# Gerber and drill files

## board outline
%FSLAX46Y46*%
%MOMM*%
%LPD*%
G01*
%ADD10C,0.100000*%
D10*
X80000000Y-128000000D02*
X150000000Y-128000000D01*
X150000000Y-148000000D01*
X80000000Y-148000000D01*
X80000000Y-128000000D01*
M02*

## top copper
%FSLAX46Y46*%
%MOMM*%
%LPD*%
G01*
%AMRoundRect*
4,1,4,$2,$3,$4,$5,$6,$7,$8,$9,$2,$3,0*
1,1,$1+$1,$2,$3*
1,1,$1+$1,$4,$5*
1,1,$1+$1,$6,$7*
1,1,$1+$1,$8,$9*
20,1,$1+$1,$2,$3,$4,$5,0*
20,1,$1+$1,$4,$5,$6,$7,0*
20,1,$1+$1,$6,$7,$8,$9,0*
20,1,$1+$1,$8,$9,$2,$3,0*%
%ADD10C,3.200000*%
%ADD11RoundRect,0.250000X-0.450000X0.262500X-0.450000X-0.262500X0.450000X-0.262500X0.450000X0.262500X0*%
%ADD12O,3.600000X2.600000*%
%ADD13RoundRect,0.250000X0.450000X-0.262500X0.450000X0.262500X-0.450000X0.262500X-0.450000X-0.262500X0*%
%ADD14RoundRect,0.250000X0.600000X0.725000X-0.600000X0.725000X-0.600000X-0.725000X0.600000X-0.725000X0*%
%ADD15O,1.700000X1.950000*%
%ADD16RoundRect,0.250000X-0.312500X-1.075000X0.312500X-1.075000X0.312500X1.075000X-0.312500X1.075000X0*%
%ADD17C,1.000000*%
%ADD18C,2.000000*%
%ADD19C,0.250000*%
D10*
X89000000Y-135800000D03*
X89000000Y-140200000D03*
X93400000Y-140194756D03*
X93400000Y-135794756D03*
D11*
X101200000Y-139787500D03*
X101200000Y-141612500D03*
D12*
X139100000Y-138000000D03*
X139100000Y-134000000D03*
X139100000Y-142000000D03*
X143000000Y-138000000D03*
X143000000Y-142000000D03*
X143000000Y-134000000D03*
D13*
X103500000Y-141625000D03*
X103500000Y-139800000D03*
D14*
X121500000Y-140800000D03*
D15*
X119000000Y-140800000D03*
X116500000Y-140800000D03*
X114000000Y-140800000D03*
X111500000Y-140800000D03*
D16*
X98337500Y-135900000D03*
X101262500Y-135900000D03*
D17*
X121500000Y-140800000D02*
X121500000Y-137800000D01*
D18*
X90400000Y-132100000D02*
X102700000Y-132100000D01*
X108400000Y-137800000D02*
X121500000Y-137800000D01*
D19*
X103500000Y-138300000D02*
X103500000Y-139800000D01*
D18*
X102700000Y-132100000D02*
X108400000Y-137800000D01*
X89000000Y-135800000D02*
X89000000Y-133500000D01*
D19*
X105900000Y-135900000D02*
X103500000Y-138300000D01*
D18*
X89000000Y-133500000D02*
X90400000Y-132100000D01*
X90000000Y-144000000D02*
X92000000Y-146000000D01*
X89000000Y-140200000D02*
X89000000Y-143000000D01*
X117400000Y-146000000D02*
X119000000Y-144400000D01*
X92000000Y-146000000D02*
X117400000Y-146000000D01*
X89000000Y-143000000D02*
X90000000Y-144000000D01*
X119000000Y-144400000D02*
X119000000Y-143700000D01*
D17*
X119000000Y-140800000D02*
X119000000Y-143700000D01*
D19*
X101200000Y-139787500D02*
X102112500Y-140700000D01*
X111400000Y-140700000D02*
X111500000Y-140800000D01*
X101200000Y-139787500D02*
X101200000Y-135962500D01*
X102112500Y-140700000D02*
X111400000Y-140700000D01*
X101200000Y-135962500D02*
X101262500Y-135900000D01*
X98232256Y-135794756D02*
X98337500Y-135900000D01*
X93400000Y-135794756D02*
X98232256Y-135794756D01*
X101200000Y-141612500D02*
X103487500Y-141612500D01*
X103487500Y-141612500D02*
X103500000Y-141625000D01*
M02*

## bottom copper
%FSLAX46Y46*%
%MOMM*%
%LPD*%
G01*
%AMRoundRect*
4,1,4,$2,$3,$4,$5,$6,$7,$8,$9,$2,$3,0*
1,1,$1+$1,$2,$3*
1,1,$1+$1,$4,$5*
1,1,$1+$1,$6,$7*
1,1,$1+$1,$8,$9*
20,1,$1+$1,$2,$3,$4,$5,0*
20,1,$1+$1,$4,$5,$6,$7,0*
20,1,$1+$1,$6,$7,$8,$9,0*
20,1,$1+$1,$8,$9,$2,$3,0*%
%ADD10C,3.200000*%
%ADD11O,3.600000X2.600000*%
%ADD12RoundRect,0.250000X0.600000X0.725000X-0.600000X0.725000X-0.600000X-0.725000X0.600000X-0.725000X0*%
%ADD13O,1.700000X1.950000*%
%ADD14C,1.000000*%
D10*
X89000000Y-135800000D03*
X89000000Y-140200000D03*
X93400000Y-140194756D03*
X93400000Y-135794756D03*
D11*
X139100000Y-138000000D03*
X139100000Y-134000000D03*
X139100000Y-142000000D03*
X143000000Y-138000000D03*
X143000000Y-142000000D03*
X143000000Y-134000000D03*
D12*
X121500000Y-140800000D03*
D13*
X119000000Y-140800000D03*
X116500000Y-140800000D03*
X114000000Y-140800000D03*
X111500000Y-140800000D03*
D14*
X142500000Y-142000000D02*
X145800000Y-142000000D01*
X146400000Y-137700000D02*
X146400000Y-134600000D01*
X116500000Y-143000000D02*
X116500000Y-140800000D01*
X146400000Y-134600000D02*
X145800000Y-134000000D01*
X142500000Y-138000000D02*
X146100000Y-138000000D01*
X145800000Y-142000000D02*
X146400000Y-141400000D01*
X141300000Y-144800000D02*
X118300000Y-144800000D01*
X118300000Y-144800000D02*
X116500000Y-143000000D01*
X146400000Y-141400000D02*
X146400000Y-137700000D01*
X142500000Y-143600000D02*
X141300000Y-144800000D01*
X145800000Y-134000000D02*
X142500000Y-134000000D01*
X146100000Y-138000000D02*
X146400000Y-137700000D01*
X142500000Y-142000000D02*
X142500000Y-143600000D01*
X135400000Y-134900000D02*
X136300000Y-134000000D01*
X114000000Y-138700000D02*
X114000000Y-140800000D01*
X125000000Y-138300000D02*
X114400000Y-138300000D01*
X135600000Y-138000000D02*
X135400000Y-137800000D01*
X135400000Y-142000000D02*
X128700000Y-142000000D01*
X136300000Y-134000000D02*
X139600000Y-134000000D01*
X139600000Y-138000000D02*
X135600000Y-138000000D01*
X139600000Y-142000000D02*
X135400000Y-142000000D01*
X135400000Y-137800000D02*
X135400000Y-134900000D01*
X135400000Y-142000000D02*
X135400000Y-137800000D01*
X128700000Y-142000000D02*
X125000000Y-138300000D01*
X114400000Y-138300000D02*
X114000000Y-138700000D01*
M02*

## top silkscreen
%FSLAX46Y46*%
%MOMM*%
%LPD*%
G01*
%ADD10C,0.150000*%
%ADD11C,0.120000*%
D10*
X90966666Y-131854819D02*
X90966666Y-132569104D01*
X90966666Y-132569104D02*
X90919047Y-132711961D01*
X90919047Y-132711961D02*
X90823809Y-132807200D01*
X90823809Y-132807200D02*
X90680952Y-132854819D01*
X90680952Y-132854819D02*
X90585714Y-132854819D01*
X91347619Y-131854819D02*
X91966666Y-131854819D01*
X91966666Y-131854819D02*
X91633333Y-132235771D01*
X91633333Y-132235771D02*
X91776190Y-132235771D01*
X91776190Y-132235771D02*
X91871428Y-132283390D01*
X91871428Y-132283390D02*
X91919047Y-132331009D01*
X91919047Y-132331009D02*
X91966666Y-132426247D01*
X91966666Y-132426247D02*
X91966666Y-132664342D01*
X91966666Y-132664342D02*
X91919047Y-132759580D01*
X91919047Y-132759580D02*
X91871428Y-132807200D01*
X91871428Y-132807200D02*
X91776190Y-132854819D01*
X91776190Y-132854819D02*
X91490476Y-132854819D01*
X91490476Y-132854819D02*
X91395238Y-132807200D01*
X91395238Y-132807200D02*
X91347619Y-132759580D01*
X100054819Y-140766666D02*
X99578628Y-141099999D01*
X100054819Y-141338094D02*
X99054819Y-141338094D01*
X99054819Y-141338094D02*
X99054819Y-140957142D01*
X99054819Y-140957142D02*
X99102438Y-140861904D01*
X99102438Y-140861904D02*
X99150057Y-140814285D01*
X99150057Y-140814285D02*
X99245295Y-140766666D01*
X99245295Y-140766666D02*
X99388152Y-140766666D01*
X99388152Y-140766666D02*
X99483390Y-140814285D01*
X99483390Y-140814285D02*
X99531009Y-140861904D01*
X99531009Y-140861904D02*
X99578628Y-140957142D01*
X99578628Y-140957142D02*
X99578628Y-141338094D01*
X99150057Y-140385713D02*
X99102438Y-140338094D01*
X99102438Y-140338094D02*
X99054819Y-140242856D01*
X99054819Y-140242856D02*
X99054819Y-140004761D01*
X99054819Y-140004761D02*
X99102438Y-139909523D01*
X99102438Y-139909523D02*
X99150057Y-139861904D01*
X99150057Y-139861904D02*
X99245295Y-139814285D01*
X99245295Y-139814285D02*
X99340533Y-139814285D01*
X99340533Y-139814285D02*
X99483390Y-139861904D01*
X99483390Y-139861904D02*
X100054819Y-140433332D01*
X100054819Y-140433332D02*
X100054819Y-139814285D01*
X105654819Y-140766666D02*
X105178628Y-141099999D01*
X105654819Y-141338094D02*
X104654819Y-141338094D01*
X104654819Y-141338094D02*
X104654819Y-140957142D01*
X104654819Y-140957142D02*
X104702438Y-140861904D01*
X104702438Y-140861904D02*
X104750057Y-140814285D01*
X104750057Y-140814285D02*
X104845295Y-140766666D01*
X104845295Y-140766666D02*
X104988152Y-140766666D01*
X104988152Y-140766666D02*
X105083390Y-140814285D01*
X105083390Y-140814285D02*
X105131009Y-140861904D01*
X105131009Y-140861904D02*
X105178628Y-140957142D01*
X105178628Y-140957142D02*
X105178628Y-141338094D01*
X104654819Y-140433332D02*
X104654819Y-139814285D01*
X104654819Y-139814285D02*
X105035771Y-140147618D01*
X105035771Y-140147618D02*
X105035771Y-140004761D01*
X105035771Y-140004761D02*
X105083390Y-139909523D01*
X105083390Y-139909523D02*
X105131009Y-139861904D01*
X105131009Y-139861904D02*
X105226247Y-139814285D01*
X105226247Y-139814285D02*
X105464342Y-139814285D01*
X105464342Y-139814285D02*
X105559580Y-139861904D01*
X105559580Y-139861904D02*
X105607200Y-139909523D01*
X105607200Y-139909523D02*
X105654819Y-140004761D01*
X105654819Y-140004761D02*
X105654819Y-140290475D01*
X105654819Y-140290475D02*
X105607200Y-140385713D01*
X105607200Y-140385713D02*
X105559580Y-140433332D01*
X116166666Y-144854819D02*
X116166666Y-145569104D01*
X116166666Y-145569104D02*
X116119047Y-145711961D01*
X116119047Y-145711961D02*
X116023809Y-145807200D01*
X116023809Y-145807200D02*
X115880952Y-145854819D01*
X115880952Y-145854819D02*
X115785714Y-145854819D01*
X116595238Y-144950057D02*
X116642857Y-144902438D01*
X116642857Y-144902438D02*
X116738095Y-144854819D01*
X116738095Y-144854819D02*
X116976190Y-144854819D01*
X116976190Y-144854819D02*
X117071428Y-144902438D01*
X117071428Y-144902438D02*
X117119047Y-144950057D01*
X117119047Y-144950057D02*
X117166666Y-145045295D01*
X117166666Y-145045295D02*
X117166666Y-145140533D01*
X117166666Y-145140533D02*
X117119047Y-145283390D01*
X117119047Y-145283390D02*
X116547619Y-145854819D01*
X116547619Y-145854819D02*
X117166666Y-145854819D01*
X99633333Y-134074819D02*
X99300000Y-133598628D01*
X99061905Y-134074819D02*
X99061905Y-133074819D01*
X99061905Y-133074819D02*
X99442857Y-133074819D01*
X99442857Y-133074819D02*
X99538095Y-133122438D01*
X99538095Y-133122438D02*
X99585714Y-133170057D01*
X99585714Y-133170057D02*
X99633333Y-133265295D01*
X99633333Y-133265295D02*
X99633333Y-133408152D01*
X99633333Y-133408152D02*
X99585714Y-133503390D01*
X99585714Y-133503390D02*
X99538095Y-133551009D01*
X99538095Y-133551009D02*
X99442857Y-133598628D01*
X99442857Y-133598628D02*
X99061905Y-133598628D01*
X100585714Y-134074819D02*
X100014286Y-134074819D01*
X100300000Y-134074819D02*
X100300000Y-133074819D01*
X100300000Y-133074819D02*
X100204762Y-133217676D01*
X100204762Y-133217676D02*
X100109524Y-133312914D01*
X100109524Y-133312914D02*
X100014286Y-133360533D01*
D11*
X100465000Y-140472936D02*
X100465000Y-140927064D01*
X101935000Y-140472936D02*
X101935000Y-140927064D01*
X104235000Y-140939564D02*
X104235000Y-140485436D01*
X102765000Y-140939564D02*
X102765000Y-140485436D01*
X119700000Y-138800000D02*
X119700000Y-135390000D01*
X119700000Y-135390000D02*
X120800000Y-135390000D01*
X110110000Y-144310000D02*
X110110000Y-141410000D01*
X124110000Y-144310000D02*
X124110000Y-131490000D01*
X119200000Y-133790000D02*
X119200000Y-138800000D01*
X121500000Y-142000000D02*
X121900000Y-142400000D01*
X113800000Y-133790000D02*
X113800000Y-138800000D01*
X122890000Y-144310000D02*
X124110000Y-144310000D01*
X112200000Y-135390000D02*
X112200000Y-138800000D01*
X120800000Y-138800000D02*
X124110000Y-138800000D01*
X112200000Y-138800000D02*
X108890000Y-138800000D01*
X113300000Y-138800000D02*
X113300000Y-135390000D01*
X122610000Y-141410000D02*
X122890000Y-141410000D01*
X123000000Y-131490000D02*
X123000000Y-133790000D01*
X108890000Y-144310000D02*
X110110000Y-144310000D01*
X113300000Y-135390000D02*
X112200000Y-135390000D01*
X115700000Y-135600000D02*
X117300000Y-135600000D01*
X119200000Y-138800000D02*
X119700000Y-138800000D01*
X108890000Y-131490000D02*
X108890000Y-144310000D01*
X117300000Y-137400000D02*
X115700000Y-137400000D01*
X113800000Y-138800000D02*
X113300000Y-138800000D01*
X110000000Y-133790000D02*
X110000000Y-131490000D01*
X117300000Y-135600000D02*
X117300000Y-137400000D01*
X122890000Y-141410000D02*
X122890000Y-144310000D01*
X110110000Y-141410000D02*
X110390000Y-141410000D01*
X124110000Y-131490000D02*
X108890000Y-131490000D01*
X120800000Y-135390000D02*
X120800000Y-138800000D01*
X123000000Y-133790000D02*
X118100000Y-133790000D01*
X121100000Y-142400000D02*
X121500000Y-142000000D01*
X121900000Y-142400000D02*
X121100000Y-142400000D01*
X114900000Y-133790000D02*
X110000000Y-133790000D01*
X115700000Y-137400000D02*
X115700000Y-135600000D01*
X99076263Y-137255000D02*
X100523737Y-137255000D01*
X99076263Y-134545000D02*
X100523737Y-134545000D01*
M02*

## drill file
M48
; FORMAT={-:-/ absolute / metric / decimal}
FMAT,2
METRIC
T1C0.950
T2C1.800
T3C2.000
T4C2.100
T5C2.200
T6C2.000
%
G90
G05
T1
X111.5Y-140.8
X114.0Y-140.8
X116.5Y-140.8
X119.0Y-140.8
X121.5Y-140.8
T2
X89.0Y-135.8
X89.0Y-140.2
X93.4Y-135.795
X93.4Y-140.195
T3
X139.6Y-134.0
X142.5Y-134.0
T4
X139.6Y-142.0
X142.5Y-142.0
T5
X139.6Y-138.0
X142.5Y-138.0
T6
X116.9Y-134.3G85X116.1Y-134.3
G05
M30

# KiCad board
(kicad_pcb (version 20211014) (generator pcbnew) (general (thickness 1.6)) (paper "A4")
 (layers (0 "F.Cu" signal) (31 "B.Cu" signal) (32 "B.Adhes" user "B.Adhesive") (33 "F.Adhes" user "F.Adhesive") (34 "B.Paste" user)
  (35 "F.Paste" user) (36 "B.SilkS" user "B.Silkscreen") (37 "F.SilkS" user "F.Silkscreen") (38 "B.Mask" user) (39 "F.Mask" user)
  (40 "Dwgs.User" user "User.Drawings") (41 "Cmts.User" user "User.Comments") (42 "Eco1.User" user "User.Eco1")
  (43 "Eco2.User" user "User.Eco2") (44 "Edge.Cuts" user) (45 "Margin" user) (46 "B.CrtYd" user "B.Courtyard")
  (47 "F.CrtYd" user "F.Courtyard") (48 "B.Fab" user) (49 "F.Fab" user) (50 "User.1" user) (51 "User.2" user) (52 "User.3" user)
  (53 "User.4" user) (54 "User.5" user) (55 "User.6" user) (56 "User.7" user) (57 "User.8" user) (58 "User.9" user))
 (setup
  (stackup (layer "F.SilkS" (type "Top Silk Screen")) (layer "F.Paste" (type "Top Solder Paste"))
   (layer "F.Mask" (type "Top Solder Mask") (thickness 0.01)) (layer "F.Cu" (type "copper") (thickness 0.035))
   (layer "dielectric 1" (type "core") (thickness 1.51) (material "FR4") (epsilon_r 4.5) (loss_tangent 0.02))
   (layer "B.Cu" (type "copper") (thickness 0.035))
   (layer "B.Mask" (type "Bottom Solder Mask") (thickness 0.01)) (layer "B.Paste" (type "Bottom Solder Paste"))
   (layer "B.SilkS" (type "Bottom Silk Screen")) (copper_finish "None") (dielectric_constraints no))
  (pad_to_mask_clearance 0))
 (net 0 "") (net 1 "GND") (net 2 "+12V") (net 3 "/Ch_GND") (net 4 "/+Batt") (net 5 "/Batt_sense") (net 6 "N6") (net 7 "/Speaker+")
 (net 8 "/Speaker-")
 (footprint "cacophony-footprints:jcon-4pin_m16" (layer "F.Cu") (at 89 135.8 -90)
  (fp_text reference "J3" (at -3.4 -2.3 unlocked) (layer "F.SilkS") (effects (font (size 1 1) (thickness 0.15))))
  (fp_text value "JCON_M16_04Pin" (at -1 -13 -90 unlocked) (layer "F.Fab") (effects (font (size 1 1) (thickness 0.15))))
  (pad "1" thru_hole circle (at 0 0 270) (size 3.2 3.2) (drill 1.8) (layers *.Cu *.Mask) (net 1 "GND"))
  (pad "2" thru_hole circle (at 4.4 0 270) (size 3.2 3.2) (drill 1.8) (layers *.Cu *.Mask) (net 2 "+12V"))
  (pad "3" thru_hole circle (at 4.394756 -4.4 270) (size 3.2 3.2) (drill 1.8) (layers *.Cu *.Mask) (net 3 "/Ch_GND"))
  (pad "4" thru_hole circle (at -0.005244 -4.4 270) (size 3.2 3.2) (drill 1.8) (layers *.Cu *.Mask) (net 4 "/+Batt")))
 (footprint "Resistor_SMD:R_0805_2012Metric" (layer "F.Cu") (at 101.2 140.7 -90)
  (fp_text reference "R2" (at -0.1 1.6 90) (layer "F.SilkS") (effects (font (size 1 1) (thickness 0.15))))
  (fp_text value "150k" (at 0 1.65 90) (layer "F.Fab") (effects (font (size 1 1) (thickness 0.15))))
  (fp_line (start -0.227064 0.735) (end 0.227064 0.735) (layer "F.SilkS") (width 0.12))
  (fp_line (start -0.227064 -0.735) (end 0.227064 -0.735) (layer "F.SilkS") (width 0.12))
  (pad "1" smd roundrect (at -0.9125 0 270) (size 1.025 1.4) (layers "F.Cu" "F.Paste" "F.Mask") (roundrect_rratio 0.243902439)
   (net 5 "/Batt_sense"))
  (pad "2" smd roundrect (at 0.9125 0 270) (size 1.025 1.4) (layers "F.Cu" "F.Paste" "F.Mask") (roundrect_rratio 0.243902439) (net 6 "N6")))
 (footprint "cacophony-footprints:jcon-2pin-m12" (layer "F.Cu") (at 142.5 138 90)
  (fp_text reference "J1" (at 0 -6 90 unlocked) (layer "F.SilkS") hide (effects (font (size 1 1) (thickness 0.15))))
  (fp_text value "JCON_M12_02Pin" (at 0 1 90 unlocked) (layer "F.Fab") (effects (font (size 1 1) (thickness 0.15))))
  (pad "1" thru_hole oval (at 0 -2.9 180) (size 3.6 2.6) (drill 2.2 (offset 0.5 0)) (layers *.Cu *.Mask) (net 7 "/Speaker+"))
  (pad "1" thru_hole oval (at 4 -2.9 180) (size 3.6 2.6) (drill 2 (offset 0.5 0)) (layers *.Cu *.Mask) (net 7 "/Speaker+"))
  (pad "1" thru_hole oval (at -4 -2.9 180) (size 3.6 2.6) (drill 2.1 (offset 0.5 0)) (layers *.Cu *.Mask) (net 7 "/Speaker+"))
  (pad "2" thru_hole oval (at 0 0) (size 3.6 2.6) (drill 2.2 (offset 0.5 0)) (layers *.Cu *.Mask) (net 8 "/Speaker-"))
  (pad "2" thru_hole oval (at -4 0) (size 3.6 2.6) (drill 2.1 (offset 0.5 0)) (layers *.Cu *.Mask) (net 8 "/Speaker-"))
  (pad "2" thru_hole oval (at 4 0) (size 3.6 2.6) (drill 2 (offset 0.5 0)) (layers *.Cu *.Mask) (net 8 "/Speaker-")))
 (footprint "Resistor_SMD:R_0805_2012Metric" (layer "F.Cu") (at 103.5 140.7125 90)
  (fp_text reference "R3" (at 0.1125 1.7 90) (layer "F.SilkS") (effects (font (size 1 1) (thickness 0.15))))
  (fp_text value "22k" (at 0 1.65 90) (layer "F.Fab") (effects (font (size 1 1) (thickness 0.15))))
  (fp_line (start -0.227064 0.735) (end 0.227064 0.735) (layer "F.SilkS") (width 0.12))
  (fp_line (start -0.227064 -0.735) (end 0.227064 -0.735) (layer "F.SilkS") (width 0.12))
  (pad "1" smd roundrect (at -0.9125 0 90) (size 1.025 1.4) (layers "F.Cu" "F.Paste" "F.Mask") (roundrect_rratio 0.243902439) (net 6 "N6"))
  (pad "2" smd roundrect (at 0.9125 0 90) (size 1.025 1.4) (layers "F.Cu" "F.Paste" "F.Mask") (roundrect_rratio 0.243902439) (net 1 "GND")))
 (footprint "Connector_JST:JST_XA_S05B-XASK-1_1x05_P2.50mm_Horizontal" (layer "F.Cu") (at 121.5 140.8 180)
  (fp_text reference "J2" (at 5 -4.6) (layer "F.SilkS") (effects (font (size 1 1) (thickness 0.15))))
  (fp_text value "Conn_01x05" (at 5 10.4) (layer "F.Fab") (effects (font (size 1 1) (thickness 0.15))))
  (fp_line (start 1.8 2) (end 1.8 5.41) (layer "F.SilkS") (width 0.12))
  (fp_line (start 1.8 5.41) (end 0.7 5.41) (layer "F.SilkS") (width 0.12))
  (fp_line (start 11.39 -3.51) (end 11.39 -0.61) (layer "F.SilkS") (width 0.12))
  (fp_line (start -2.61 -3.51) (end -2.61 9.31) (layer "F.SilkS") (width 0.12))
  (fp_line (start 2.3 7.01) (end 2.3 2) (layer "F.SilkS") (width 0.12))
  (fp_line (start 0 -1.2) (end -0.4 -1.6) (layer "F.SilkS") (width 0.12))
  (fp_line (start 7.7 7.01) (end 7.7 2) (layer "F.SilkS") (width 0.12))
  (fp_line (start -1.39 -3.51) (end -2.61 -3.51) (layer "F.SilkS") (width 0.12))
  (fp_line (start 9.3 5.41) (end 9.3 2) (layer "F.SilkS") (width 0.12))
  (fp_line (start 0.7 2) (end -2.61 2) (layer "F.SilkS") (width 0.12))
  (fp_line (start 9.3 2) (end 12.61 2) (layer "F.SilkS") (width 0.12))
  (fp_line (start 8.2 2) (end 8.2 5.41) (layer "F.SilkS") (width 0.12))
  (fp_line (start -1.11 -0.61) (end -1.39 -0.61) (layer "F.SilkS") (width 0.12))
  (fp_line (start -1.5 9.31) (end -1.5 7.01) (layer "F.SilkS") (width 0.12))
  (fp_line (start 12.61 -3.51) (end 11.39 -3.51) (layer "F.SilkS") (width 0.12))
  (fp_line (start 8.2 5.41) (end 9.3 5.41) (layer "F.SilkS") (width 0.12))
  (fp_line (start 5.8 5.2) (end 4.2 5.2) (layer "F.SilkS") (width 0.12))
  (fp_line (start 2.3 2) (end 1.8 2) (layer "F.SilkS") (width 0.12))
  (fp_line (start 12.61 9.31) (end 12.61 -3.51) (layer "F.SilkS") (width 0.12))
  (fp_line (start 4.2 3.4) (end 5.8 3.4) (layer "F.SilkS") (width 0.12))
  (fp_line (start 7.7 2) (end 8.2 2) (layer "F.SilkS") (width 0.12))
  (fp_line (start 11.5 7.01) (end 11.5 9.31) (layer "F.SilkS") (width 0.12))
  (fp_line (start 4.2 5.2) (end 4.2 3.4) (layer "F.SilkS") (width 0.12))
  (fp_line (start -1.39 -0.61) (end -1.39 -3.51) (layer "F.SilkS") (width 0.12))
  (fp_line (start 11.39 -0.61) (end 11.11 -0.61) (layer "F.SilkS") (width 0.12))
  (fp_line (start -2.61 9.31) (end 12.61 9.31) (layer "F.SilkS") (width 0.12))
  (fp_line (start 0.7 5.41) (end 0.7 2) (layer "F.SilkS") (width 0.12))
  (fp_line (start -1.5 7.01) (end 3.4 7.01) (layer "F.SilkS") (width 0.12))
  (fp_line (start 0.4 -1.6) (end 0 -1.2) (layer "F.SilkS") (width 0.12))
  (fp_line (start -0.4 -1.6) (end 0.4 -1.6) (layer "F.SilkS") (width 0.12))
  (fp_line (start 6.6 7.01) (end 11.5 7.01) (layer "F.SilkS") (width 0.12))
  (fp_line (start 5.8 3.4) (end 5.8 5.2) (layer "F.SilkS") (width 0.12))
  (pad "" np_thru_hole oval (at 5 6.5 180) (size 2.8 2) (drill oval 2.8 2) (layers *.Cu *.Mask))
  (pad "1" thru_hole roundrect (at 0 0 180) (size 1.7 1.95) (drill 0.95) (layers *.Cu *.Mask) (roundrect_rratio 0.1470588235) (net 1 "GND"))
  (pad "2" thru_hole oval (at 2.5 0 180) (size 1.7 1.95) (drill 0.95) (layers *.Cu *.Mask) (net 2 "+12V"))
  (pad "3" thru_hole oval (at 5 0 180) (size 1.7 1.95) (drill 0.95) (layers *.Cu *.Mask) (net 8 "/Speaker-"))
  (pad "4" thru_hole oval (at 7.5 0 180) (size 1.7 1.95) (drill 0.95) (layers *.Cu *.Mask) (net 7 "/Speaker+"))
  (pad "5" thru_hole oval (at 10 0 180) (size 1.7 1.95) (drill 0.95) (layers *.Cu *.Mask) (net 5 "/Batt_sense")))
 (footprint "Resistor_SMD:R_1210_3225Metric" (layer "F.Cu") (at 99.8 135.9)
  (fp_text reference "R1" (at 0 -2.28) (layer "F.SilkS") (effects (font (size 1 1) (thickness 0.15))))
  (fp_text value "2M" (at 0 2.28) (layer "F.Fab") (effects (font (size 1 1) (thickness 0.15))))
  (fp_line (start -0.723737 1.355) (end 0.723737 1.355) (layer "F.SilkS") (width 0.12))
  (fp_line (start -0.723737 -1.355) (end 0.723737 -1.355) (layer "F.SilkS") (width 0.12))
  (pad "1" smd roundrect (at -1.4625 0) (size 1.125 2.65) (layers "F.Cu" "F.Paste" "F.Mask") (roundrect_rratio 0.2222222222)
   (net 4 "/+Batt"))
  (pad "2" smd roundrect (at 1.4625 0) (size 1.125 2.65) (layers "F.Cu" "F.Paste" "F.Mask") (roundrect_rratio 0.2222222222)
   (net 5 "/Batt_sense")))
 (gr_rect (start 80 148) (end 150 128) (layer "Edge.Cuts") (width 0.1) (fill none))
 (segment (start 121.5 140.8) (end 121.5 137.8) (width 1) (layer "F.Cu") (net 1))
 (segment (start 90.4 132.1) (end 102.7 132.1) (width 2) (layer "F.Cu") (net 1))
 (segment (start 108.4 137.8) (end 121.5 137.8) (width 2) (layer "F.Cu") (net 1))
 (segment (start 103.5 138.3) (end 103.5 139.8) (width 0.25) (layer "F.Cu") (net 1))
 (segment (start 102.7 132.1) (end 108.4 137.8) (width 2) (layer "F.Cu") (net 1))
 (segment (start 89 135.8) (end 89 133.5) (width 2) (layer "F.Cu") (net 1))
 (segment (start 105.9 135.9) (end 103.5 138.3) (width 0.25) (layer "F.Cu") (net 1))
 (segment (start 89 133.5) (end 90.4 132.1) (width 2) (layer "F.Cu") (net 1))
 (segment (start 90 144) (end 92 146) (width 2) (layer "F.Cu") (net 2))
 (segment (start 89 140.2) (end 89 143) (width 2) (layer "F.Cu") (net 2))
 (segment (start 117.4 146) (end 119 144.4) (width 2) (layer "F.Cu") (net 2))
 (segment (start 92 146) (end 117.4 146) (width 2) (layer "F.Cu") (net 2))
 (segment (start 89 143) (end 90 144) (width 2) (layer "F.Cu") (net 2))
 (segment (start 119 144.4) (end 119 143.7) (width 2) (layer "F.Cu") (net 2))
 (segment (start 119 140.8) (end 119 143.7) (width 1) (layer "F.Cu") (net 2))
 (segment (start 142.5 142) (end 145.8 142) (width 1) (layer "B.Cu") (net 8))
 (segment (start 146.4 137.7) (end 146.4 134.6) (width 1) (layer "B.Cu") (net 8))
 (segment (start 116.5 143) (end 116.5 140.8) (width 1) (layer "B.Cu") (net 8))
 (segment (start 146.4 134.6) (end 145.8 134) (width 1) (layer "B.Cu") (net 8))
 (segment (start 142.5 138) (end 146.1 138) (width 1) (layer "B.Cu") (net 8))
 (segment (start 145.8 142) (end 146.4 141.4) (width 1) (layer "B.Cu") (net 8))
 (segment (start 141.3 144.8) (end 118.3 144.8) (width 1) (layer "B.Cu") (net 8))
 (segment (start 118.3 144.8) (end 116.5 143) (width 1) (layer "B.Cu") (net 8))
 (segment (start 146.4 141.4) (end 146.4 137.7) (width 1) (layer "B.Cu") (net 8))
 (segment (start 142.5 143.6) (end 141.3 144.8) (width 1) (layer "B.Cu") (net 8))
 (segment (start 145.8 134) (end 142.5 134) (width 1) (layer "B.Cu") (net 8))
 (segment (start 146.1 138) (end 146.4 137.7) (width 1) (layer "B.Cu") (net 8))
 (segment (start 142.5 142) (end 142.5 143.6) (width 1) (layer "B.Cu") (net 8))
 (segment (start 135.4 134.9) (end 136.3 134) (width 1) (layer "B.Cu") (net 7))
 (segment (start 114 138.7) (end 114 140.8) (width 1) (layer "B.Cu") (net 7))
 (segment (start 125 138.3) (end 114.4 138.3) (width 1) (layer "B.Cu") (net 7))
 (segment (start 135.6 138) (end 135.4 137.8) (width 1) (layer "B.Cu") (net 7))
 (segment (start 135.4 142) (end 128.7 142) (width 1) (layer "B.Cu") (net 7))
 (segment (start 136.3 134) (end 139.6 134) (width 1) (layer "B.Cu") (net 7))
 (segment (start 139.6 138) (end 135.6 138) (width 1) (layer "B.Cu") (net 7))
 (segment (start 139.6 142) (end 135.4 142) (width 1) (layer "B.Cu") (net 7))
 (segment (start 135.4 137.8) (end 135.4 134.9) (width 1) (layer "B.Cu") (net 7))
 (segment (start 135.4 142) (end 135.4 137.8) (width 1) (layer "B.Cu") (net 7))
 (segment (start 128.7 142) (end 125 138.3) (width 1) (layer "B.Cu") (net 7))
 (segment (start 114.4 138.3) (end 114 138.7) (width 1) (layer "B.Cu") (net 7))
 (segment (start 101.2 139.7875) (end 102.1125 140.7) (width 0.25) (layer "F.Cu") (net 5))
 (segment (start 111.4 140.7) (end 111.5 140.8) (width 0.25) (layer "F.Cu") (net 5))
 (segment (start 101.2 139.7875) (end 101.2 135.9625) (width 0.25) (layer "F.Cu") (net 5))
 (segment (start 102.1125 140.7) (end 111.4 140.7) (width 0.25) (layer "F.Cu") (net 5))
 (segment (start 101.2 135.9625) (end 101.2625 135.9) (width 0.25) (layer "F.Cu") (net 5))
 (segment (start 98.232256 135.794756) (end 98.3375 135.9) (width 0.25) (layer "F.Cu") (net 4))
 (segment (start 93.4 135.794756) (end 98.232256 135.794756) (width 0.25) (layer "F.Cu") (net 4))
 (segment (start 101.2 141.6125) (end 103.4875 141.6125) (width 0.25) (layer "F.Cu") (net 6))
 (segment (start 103.4875 141.6125) (end 103.5 141.625) (width 0.25) (layer "F.Cu") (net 6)))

